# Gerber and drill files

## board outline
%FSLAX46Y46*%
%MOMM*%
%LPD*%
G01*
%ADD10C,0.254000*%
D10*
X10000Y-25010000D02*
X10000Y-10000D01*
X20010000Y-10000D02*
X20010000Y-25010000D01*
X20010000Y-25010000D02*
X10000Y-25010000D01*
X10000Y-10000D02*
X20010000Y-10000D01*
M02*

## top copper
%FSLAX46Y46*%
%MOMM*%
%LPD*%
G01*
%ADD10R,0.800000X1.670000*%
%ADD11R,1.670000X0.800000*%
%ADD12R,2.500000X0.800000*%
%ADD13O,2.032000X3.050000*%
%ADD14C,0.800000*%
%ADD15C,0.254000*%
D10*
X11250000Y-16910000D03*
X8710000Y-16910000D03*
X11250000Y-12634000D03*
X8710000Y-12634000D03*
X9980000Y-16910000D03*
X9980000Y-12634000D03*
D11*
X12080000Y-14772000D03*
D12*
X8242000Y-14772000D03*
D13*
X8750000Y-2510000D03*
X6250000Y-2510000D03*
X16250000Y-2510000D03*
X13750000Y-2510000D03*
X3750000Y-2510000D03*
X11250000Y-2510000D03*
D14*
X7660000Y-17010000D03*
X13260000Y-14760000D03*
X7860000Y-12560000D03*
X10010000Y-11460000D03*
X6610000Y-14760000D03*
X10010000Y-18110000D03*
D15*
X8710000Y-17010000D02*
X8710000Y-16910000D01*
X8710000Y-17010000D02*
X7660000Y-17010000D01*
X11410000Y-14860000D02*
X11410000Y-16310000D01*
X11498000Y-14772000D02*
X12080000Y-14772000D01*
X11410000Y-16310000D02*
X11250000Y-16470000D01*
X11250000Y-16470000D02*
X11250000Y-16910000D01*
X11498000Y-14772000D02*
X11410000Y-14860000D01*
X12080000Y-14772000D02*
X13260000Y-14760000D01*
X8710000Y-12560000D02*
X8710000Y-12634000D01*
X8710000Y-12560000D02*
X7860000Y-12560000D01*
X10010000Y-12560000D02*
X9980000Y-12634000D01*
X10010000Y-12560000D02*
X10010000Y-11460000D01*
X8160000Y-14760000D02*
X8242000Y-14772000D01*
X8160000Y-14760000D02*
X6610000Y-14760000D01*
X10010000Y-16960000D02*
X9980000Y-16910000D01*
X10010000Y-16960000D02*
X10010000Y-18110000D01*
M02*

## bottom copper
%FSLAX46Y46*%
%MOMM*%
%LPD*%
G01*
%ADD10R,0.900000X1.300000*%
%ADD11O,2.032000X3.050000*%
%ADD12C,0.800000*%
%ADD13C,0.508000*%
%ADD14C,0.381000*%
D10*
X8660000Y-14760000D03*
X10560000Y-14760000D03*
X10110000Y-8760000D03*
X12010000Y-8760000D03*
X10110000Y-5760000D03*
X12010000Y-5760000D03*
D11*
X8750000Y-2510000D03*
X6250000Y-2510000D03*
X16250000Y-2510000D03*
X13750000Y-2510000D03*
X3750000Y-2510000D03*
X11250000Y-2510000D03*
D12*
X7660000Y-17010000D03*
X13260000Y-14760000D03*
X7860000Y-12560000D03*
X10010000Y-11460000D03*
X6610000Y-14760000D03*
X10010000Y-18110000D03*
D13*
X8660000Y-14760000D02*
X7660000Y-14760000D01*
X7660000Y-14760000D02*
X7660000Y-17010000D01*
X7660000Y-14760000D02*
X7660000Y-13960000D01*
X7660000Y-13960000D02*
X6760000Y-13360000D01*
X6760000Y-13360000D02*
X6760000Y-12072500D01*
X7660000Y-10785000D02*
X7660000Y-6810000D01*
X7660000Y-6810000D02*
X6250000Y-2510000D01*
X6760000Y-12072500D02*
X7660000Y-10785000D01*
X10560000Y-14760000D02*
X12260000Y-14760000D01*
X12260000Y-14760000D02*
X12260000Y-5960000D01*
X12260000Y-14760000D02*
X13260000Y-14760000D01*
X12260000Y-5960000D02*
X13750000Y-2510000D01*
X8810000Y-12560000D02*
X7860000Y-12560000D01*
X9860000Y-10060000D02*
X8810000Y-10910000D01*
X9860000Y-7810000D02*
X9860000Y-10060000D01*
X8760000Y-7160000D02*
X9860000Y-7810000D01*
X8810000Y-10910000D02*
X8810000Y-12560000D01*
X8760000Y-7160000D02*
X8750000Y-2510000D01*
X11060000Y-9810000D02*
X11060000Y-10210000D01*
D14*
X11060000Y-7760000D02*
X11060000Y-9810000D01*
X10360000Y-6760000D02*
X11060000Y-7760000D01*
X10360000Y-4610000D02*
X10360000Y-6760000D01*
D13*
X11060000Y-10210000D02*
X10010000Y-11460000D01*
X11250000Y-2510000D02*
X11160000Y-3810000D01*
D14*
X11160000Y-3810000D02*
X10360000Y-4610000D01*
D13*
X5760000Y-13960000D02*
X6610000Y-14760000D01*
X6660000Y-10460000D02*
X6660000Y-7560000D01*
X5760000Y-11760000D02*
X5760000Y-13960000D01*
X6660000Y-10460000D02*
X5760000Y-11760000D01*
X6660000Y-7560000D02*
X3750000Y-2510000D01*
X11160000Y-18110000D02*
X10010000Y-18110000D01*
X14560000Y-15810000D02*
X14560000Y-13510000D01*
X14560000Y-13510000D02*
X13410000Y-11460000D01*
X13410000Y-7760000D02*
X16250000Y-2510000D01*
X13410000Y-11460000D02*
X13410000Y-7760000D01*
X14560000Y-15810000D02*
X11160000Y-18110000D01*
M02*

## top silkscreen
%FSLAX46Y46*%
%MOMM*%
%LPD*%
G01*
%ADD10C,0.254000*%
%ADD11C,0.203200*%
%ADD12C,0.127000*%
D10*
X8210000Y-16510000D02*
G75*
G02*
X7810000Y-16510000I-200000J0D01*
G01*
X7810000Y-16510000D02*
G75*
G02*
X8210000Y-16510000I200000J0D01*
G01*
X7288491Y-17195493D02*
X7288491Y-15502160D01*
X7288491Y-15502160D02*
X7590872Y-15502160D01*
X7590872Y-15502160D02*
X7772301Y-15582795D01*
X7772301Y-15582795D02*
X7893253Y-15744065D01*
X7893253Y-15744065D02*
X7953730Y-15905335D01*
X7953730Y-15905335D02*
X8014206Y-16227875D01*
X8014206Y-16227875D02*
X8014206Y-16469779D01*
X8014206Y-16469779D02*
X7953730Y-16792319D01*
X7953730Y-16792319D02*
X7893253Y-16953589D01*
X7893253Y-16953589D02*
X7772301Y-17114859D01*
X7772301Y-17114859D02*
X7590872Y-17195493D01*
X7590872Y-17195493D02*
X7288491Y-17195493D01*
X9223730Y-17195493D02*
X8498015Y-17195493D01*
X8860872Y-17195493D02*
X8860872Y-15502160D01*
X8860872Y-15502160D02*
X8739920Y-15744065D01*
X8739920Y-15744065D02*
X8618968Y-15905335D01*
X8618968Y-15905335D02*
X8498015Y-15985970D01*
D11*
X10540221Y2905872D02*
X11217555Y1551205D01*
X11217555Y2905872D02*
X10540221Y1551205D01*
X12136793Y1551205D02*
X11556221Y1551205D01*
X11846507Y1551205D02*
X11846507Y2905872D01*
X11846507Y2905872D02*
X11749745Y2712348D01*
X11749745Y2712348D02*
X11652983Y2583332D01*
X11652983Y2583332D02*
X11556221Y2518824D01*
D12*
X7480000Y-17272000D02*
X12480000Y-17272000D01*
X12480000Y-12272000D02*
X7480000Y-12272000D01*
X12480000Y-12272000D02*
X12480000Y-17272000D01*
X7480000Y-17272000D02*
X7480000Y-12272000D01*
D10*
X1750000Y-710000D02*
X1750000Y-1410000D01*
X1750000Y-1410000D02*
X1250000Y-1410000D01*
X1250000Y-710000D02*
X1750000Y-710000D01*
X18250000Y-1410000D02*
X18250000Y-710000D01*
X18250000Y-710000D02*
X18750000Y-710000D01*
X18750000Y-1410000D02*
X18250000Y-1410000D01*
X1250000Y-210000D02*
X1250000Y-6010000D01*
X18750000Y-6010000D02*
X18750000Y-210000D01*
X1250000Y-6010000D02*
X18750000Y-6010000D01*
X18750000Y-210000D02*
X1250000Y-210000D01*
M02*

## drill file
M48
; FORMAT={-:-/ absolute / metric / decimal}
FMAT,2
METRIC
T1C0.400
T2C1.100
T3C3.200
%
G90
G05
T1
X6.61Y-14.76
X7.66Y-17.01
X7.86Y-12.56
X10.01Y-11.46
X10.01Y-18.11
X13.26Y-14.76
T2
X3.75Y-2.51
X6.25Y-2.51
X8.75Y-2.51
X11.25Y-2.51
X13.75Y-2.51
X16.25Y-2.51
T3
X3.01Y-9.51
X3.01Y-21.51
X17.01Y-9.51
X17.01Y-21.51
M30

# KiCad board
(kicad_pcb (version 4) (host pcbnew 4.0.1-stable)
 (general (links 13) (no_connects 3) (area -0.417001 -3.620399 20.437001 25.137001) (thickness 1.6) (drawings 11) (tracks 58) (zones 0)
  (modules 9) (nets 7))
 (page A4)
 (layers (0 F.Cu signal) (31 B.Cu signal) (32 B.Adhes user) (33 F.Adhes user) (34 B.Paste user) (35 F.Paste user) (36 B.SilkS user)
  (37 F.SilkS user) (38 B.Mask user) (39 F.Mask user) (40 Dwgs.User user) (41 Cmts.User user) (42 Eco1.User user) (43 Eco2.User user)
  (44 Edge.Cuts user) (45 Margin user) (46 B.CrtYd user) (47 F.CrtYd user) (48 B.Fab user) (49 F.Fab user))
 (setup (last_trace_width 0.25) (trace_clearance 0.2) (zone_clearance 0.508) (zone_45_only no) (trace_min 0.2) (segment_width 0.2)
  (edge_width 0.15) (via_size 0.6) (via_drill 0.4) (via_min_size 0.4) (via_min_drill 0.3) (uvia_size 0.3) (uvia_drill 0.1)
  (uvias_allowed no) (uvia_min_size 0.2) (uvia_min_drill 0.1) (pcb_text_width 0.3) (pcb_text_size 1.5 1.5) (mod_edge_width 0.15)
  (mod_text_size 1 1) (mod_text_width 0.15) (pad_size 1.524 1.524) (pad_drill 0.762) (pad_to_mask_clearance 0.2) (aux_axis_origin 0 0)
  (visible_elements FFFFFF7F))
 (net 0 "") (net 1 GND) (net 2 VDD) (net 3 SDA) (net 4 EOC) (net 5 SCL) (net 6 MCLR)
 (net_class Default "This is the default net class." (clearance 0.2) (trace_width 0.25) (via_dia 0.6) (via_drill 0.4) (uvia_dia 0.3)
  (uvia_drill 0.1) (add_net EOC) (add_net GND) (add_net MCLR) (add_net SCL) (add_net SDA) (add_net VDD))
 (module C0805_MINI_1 (layer B.Cu) (at 10.56 14.76)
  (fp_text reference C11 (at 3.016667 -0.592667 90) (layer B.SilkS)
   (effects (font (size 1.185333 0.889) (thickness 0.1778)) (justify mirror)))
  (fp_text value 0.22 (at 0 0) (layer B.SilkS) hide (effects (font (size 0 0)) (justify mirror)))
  (pad 2 smd rect (at -1.9 0) (size 0.9 1.3) (layers B.Cu B.Paste B.Mask) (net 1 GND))
  (pad 1 smd rect (at 0 0) (size 0.9 1.3) (layers B.Cu B.Paste B.Mask) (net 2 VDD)))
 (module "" (layer F.Cu) (at 17.01 21.51)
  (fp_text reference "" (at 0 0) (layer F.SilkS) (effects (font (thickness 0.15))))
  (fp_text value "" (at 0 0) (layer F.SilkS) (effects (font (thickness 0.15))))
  (pad "" np_thru_hole circle (at 0 0) (size 3.2 3.2) (drill 3.2) (layers *.Cu *.Mask)))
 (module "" (layer F.Cu) (at 17.01 9.51)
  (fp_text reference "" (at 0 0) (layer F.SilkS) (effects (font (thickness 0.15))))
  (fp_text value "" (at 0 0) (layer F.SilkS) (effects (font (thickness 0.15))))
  (pad "" np_thru_hole circle (at 0 0) (size 3.2 3.2) (drill 3.2) (layers *.Cu *.Mask)))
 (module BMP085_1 (layer F.Cu) (at 8.71 16.51 90)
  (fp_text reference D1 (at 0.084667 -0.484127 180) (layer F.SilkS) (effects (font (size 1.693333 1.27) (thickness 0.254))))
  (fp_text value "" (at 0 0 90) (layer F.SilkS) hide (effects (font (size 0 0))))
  (fp_line (start -0.762 -1.23) (end -0.762 3.77) (layer F.SilkS) (width 0.127))
  (fp_line (start 4.238 3.77) (end 4.238 -1.23) (layer F.SilkS) (width 0.127))
  (fp_line (start 4.238 3.77) (end -0.762 3.77) (layer F.SilkS) (width 0.127))
  (fp_line (start -0.762 -1.23) (end 4.238 -1.23) (layer F.SilkS) (width 0.127))
  (pad 3 smd rect (at -0.4 2.54 180) (size 0.8 1.67) (layers F.Cu F.Paste F.Mask) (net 2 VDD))
  (pad 1 smd rect (at -0.4 0 180) (size 0.8 1.67) (layers F.Cu F.Paste F.Mask) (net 1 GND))
  (pad 5 smd rect (at 3.876 2.54 180) (size 0.8 1.67) (layers F.Cu F.Paste F.Mask))
  (pad 7 smd rect (at 3.876 0 180) (size 0.8 1.67) (layers F.Cu F.Paste F.Mask) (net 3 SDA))
  (pad 2 smd rect (at -0.4 1.27 180) (size 0.8 1.67) (layers F.Cu F.Paste F.Mask) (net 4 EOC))
  (pad 6 smd rect (at 3.876 1.27 180) (size 0.8 1.67) (layers F.Cu F.Paste F.Mask) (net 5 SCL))
  (pad 4 smd rect (at 1.738 3.37 90) (size 0.8 1.67) (layers F.Cu F.Paste F.Mask) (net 2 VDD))
  (pad 8 smd rect (at 1.738 -0.468 90) (size 0.8 2.5) (layers F.Cu F.Paste F.Mask) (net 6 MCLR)))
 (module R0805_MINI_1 (layer B.Cu) (at 12.01 8.76)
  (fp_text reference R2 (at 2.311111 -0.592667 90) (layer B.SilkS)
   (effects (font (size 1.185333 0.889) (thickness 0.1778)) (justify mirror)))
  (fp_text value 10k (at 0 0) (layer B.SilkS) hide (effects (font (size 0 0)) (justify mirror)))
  (pad 2 smd rect (at -1.9 0) (size 0.9 1.3) (layers B.Cu B.Paste B.Mask) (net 3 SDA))
  (pad 1 smd rect (at 0 0) (size 0.9 1.3) (layers B.Cu B.Paste B.Mask) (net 2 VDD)))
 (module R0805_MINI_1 (layer B.Cu) (at 12.01 5.76)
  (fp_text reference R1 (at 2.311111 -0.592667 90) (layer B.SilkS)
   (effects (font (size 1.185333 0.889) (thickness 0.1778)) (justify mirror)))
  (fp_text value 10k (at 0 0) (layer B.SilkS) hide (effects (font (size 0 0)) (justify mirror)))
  (pad 2 smd rect (at -1.9 0) (size 0.9 1.3) (layers B.Cu B.Paste B.Mask) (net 5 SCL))
  (pad 1 smd rect (at 0 0) (size 0.9 1.3) (layers B.Cu B.Paste B.Mask) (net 2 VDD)))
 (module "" (layer F.Cu) (at 3.01 21.51)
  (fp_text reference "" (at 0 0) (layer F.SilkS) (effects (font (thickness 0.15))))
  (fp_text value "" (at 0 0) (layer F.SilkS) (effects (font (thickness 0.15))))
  (pad "" np_thru_hole circle (at 0 0) (size 3.2 3.2) (drill 3.2) (layers *.Cu *.Mask)))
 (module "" (layer F.Cu) (at 3.01 9.51)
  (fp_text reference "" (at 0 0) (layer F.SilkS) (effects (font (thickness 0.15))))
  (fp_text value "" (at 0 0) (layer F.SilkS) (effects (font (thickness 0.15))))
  (pad "" np_thru_hole circle (at 0 0) (size 3.2 3.2) (drill 3.2) (layers *.Cu *.Mask)))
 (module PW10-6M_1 (layer F.Cu) (at 3.71 2.51)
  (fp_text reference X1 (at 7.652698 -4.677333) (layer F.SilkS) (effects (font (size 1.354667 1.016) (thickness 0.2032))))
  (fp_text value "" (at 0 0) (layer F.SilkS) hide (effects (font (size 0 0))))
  (fp_line (start -1.96 -1.8) (end -1.96 -1.1) (layer F.SilkS) (width 0.254))
  (fp_line (start -1.96 -1.1) (end -2.46 -1.1) (layer F.SilkS) (width 0.254))
  (fp_line (start -2.46 -1.8) (end -1.96 -1.8) (layer F.SilkS) (width 0.254))
  (fp_line (start 14.54 -1.1) (end 14.54 -1.8) (layer F.SilkS) (width 0.254))
  (fp_line (start 14.54 -1.8) (end 15.04 -1.8) (layer F.SilkS) (width 0.254))
  (fp_line (start 15.04 -1.1) (end 14.54 -1.1) (layer F.SilkS) (width 0.254))
  (fp_line (start -2.46 -2.3) (end -2.46 3.5) (layer F.SilkS) (width 0.254))
  (fp_line (start 15.04 3.5) (end 15.04 -2.3) (layer F.SilkS) (width 0.254))
  (fp_line (start -2.46 3.5) (end 15.04 3.5) (layer F.SilkS) (width 0.254))
  (fp_line (start 15.04 -2.3) (end -2.46 -2.3) (layer F.SilkS) (width 0.254))
  (pad 3 thru_hole oval (at 5.04 0 90) (size 3.05 2.032) (drill 1.1) (layers *.Cu *.Mask) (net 3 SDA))
  (pad 2 thru_hole oval (at 2.54 0 90) (size 3.05 2.032) (drill 1.1) (layers *.Cu *.Mask) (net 1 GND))
  (pad 6 thru_hole oval (at 12.54 0 90) (size 3.05 2.032) (drill 1.1) (layers *.Cu *.Mask) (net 4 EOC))
  (pad 5 thru_hole oval (at 10.04 0 90) (size 3.05 2.032) (drill 1.1) (layers *.Cu *.Mask) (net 2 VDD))
  (pad 1 thru_hole oval (at 0.04 0 90) (size 3.05 2.032) (drill 1.1) (layers *.Cu *.Mask) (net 6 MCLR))
  (pad 4 thru_hole oval (at 7.54 0 90) (size 3.05 2.032) (drill 1.1) (layers *.Cu *.Mask) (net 5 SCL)))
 (gr_line (start 0.01 25.01) (end 0.01 0.01) (layer Edge.Cuts) (width 0.254))
 (gr_line (start 20.01 0.01) (end 20.01 25.01) (layer Edge.Cuts) (width 0.254))
 (gr_line (start 20.01 25.01) (end 0.01 25.01) (layer Edge.Cuts) (width 0.254))
 (gr_line (start 0.01 0.01) (end 20.01 0.01) (layer Edge.Cuts) (width 0.254))
 (gr_arc (start 8.01 16.51) (end 7.81 16.51) (angle -360) (layer F.SilkS) (width 0.254))
 (via (at 7.66 17.01) (size 0.8) (drill 0.4) (layers F.Cu B.Cu) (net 1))
 (segment (start 8.71 17.01) (end 8.71 16.91) (width 0.254) (layer F.Cu) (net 1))
 (segment (start 8.71 17.01) (end 7.66 17.01) (width 0.254) (layer F.Cu) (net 1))
 (segment (start 8.66 14.76) (end 7.66 14.76) (width 0.508) (layer B.Cu) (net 1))
 (segment (start 7.66 14.76) (end 7.66 17.01) (width 0.508) (layer B.Cu) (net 1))
 (segment (start 7.66 14.76) (end 7.66 13.96) (width 0.508) (layer B.Cu) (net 1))
 (segment (start 7.66 13.96) (end 6.76 13.36) (width 0.508) (layer B.Cu) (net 1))
 (segment (start 6.76 13.36) (end 6.76 12.0725) (width 0.508) (layer B.Cu) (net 1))
 (segment (start 7.66 10.785) (end 7.66 6.81) (width 0.508) (layer B.Cu) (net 1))
 (segment (start 7.66 6.81) (end 6.25 2.51) (width 0.508) (layer B.Cu) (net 1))
 (segment (start 6.76 12.0725) (end 7.66 10.785) (width 0.508) (layer B.Cu) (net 1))
 (via (at 13.26 14.76) (size 0.8) (drill 0.4) (layers F.Cu B.Cu) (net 2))
 (segment (start 11.41 14.86) (end 11.41 16.31) (width 0.254) (layer F.Cu) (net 2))
 (segment (start 11.498 14.772) (end 12.08 14.772) (width 0.254) (layer F.Cu) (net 2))
 (segment (start 11.41 16.31) (end 11.25 16.47) (width 0.254) (layer F.Cu) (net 2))
 (segment (start 11.25 16.47) (end 11.25 16.91) (width 0.254) (layer F.Cu) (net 2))
 (segment (start 11.498 14.772) (end 11.41 14.86) (width 0.254) (layer F.Cu) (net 2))
 (segment (start 12.08 14.772) (end 13.26 14.76) (width 0.254) (layer F.Cu) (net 2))
 (segment (start 10.56 14.76) (end 12.26 14.76) (width 0.508) (layer B.Cu) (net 2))
 (segment (start 12.26 14.76) (end 12.26 5.96) (width 0.508) (layer B.Cu) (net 2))
 (segment (start 12.26 14.76) (end 13.26 14.76) (width 0.508) (layer B.Cu) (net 2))
 (segment (start 12.26 5.96) (end 13.75 2.51) (width 0.508) (layer B.Cu) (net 2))
 (via (at 7.86 12.56) (size 0.8) (drill 0.4) (layers F.Cu B.Cu) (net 3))
 (segment (start 8.71 12.56) (end 8.71 12.634) (width 0.254) (layer F.Cu) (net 3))
 (segment (start 8.71 12.56) (end 7.86 12.56) (width 0.254) (layer F.Cu) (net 3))
 (segment (start 8.81 12.56) (end 7.86 12.56) (width 0.508) (layer B.Cu) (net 3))
 (segment (start 9.86 10.06) (end 8.81 10.91) (width 0.508) (layer B.Cu) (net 3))
 (segment (start 9.86 7.81) (end 9.86 10.06) (width 0.508) (layer B.Cu) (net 3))
 (segment (start 8.76 7.16) (end 9.86 7.81) (width 0.508) (layer B.Cu) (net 3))
 (segment (start 8.81 10.91) (end 8.81 12.56) (width 0.508) (layer B.Cu) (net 3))
 (segment (start 8.76 7.16) (end 8.75 2.51) (width 0.508) (layer B.Cu) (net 3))
 (via (at 10.01 11.46) (size 0.8) (drill 0.4) (layers F.Cu B.Cu) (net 5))
 (segment (start 10.01 12.56) (end 9.98 12.634) (width 0.254) (layer F.Cu) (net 5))
 (segment (start 10.01 12.56) (end 10.01 11.46) (width 0.254) (layer F.Cu) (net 5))
 (segment (start 11.06 9.81) (end 11.06 10.21) (width 0.508) (layer B.Cu) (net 5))
 (segment (start 11.06 7.76) (end 11.06 9.81) (width 0.381) (layer B.Cu) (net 5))
 (segment (start 10.36 6.76) (end 11.06 7.76) (width 0.381) (layer B.Cu) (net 5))
 (segment (start 10.36 4.61) (end 10.36 6.76) (width 0.381) (layer B.Cu) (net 5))
 (segment (start 11.06 10.21) (end 10.01 11.46) (width 0.508) (layer B.Cu) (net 5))
 (segment (start 11.25 2.51) (end 11.16 3.81) (width 0.508) (layer B.Cu) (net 5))
 (segment (start 11.16 3.81) (end 10.36 4.61) (width 0.381) (layer B.Cu) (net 5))
 (via (at 6.61 14.76) (size 0.8) (drill 0.4) (layers F.Cu B.Cu) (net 6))
 (segment (start 8.16 14.76) (end 8.242 14.772) (width 0.254) (layer F.Cu) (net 6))
 (segment (start 8.16 14.76) (end 6.61 14.76) (width 0.254) (layer F.Cu) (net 6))
 (segment (start 5.76 13.96) (end 6.61 14.76) (width 0.508) (layer B.Cu) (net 6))
 (segment (start 6.66 10.46) (end 6.66 7.56) (width 0.508) (layer B.Cu) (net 6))
 (segment (start 5.76 11.76) (end 5.76 13.96) (width 0.508) (layer B.Cu) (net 6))
 (segment (start 6.66 10.46) (end 5.76 11.76) (width 0.508) (layer B.Cu) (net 6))
 (segment (start 6.66 7.56) (end 3.75 2.51) (width 0.508) (layer B.Cu) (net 6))
 (via (at 10.01 18.11) (size 0.8) (drill 0.4) (layers F.Cu B.Cu) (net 4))
 (segment (start 10.01 16.96) (end 9.98 16.91) (width 0.254) (layer F.Cu) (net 4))
 (segment (start 10.01 16.96) (end 10.01 18.11) (width 0.254) (layer F.Cu) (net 4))
 (segment (start 11.16 18.11) (end 10.01 18.11) (width 0.508) (layer B.Cu) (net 4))
 (segment (start 14.56 15.81) (end 14.56 13.51) (width 0.508) (layer B.Cu) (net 4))
 (segment (start 14.56 13.51) (end 13.41 11.46) (width 0.508) (layer B.Cu) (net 4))
 (segment (start 13.41 7.76) (end 16.25 2.51) (width 0.508) (layer B.Cu) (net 4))
 (segment (start 13.41 11.46) (end 13.41 7.76) (width 0.508) (layer B.Cu) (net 4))
 (segment (start 14.56 15.81) (end 11.16 18.11) (width 0.508) (layer B.Cu) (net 4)))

